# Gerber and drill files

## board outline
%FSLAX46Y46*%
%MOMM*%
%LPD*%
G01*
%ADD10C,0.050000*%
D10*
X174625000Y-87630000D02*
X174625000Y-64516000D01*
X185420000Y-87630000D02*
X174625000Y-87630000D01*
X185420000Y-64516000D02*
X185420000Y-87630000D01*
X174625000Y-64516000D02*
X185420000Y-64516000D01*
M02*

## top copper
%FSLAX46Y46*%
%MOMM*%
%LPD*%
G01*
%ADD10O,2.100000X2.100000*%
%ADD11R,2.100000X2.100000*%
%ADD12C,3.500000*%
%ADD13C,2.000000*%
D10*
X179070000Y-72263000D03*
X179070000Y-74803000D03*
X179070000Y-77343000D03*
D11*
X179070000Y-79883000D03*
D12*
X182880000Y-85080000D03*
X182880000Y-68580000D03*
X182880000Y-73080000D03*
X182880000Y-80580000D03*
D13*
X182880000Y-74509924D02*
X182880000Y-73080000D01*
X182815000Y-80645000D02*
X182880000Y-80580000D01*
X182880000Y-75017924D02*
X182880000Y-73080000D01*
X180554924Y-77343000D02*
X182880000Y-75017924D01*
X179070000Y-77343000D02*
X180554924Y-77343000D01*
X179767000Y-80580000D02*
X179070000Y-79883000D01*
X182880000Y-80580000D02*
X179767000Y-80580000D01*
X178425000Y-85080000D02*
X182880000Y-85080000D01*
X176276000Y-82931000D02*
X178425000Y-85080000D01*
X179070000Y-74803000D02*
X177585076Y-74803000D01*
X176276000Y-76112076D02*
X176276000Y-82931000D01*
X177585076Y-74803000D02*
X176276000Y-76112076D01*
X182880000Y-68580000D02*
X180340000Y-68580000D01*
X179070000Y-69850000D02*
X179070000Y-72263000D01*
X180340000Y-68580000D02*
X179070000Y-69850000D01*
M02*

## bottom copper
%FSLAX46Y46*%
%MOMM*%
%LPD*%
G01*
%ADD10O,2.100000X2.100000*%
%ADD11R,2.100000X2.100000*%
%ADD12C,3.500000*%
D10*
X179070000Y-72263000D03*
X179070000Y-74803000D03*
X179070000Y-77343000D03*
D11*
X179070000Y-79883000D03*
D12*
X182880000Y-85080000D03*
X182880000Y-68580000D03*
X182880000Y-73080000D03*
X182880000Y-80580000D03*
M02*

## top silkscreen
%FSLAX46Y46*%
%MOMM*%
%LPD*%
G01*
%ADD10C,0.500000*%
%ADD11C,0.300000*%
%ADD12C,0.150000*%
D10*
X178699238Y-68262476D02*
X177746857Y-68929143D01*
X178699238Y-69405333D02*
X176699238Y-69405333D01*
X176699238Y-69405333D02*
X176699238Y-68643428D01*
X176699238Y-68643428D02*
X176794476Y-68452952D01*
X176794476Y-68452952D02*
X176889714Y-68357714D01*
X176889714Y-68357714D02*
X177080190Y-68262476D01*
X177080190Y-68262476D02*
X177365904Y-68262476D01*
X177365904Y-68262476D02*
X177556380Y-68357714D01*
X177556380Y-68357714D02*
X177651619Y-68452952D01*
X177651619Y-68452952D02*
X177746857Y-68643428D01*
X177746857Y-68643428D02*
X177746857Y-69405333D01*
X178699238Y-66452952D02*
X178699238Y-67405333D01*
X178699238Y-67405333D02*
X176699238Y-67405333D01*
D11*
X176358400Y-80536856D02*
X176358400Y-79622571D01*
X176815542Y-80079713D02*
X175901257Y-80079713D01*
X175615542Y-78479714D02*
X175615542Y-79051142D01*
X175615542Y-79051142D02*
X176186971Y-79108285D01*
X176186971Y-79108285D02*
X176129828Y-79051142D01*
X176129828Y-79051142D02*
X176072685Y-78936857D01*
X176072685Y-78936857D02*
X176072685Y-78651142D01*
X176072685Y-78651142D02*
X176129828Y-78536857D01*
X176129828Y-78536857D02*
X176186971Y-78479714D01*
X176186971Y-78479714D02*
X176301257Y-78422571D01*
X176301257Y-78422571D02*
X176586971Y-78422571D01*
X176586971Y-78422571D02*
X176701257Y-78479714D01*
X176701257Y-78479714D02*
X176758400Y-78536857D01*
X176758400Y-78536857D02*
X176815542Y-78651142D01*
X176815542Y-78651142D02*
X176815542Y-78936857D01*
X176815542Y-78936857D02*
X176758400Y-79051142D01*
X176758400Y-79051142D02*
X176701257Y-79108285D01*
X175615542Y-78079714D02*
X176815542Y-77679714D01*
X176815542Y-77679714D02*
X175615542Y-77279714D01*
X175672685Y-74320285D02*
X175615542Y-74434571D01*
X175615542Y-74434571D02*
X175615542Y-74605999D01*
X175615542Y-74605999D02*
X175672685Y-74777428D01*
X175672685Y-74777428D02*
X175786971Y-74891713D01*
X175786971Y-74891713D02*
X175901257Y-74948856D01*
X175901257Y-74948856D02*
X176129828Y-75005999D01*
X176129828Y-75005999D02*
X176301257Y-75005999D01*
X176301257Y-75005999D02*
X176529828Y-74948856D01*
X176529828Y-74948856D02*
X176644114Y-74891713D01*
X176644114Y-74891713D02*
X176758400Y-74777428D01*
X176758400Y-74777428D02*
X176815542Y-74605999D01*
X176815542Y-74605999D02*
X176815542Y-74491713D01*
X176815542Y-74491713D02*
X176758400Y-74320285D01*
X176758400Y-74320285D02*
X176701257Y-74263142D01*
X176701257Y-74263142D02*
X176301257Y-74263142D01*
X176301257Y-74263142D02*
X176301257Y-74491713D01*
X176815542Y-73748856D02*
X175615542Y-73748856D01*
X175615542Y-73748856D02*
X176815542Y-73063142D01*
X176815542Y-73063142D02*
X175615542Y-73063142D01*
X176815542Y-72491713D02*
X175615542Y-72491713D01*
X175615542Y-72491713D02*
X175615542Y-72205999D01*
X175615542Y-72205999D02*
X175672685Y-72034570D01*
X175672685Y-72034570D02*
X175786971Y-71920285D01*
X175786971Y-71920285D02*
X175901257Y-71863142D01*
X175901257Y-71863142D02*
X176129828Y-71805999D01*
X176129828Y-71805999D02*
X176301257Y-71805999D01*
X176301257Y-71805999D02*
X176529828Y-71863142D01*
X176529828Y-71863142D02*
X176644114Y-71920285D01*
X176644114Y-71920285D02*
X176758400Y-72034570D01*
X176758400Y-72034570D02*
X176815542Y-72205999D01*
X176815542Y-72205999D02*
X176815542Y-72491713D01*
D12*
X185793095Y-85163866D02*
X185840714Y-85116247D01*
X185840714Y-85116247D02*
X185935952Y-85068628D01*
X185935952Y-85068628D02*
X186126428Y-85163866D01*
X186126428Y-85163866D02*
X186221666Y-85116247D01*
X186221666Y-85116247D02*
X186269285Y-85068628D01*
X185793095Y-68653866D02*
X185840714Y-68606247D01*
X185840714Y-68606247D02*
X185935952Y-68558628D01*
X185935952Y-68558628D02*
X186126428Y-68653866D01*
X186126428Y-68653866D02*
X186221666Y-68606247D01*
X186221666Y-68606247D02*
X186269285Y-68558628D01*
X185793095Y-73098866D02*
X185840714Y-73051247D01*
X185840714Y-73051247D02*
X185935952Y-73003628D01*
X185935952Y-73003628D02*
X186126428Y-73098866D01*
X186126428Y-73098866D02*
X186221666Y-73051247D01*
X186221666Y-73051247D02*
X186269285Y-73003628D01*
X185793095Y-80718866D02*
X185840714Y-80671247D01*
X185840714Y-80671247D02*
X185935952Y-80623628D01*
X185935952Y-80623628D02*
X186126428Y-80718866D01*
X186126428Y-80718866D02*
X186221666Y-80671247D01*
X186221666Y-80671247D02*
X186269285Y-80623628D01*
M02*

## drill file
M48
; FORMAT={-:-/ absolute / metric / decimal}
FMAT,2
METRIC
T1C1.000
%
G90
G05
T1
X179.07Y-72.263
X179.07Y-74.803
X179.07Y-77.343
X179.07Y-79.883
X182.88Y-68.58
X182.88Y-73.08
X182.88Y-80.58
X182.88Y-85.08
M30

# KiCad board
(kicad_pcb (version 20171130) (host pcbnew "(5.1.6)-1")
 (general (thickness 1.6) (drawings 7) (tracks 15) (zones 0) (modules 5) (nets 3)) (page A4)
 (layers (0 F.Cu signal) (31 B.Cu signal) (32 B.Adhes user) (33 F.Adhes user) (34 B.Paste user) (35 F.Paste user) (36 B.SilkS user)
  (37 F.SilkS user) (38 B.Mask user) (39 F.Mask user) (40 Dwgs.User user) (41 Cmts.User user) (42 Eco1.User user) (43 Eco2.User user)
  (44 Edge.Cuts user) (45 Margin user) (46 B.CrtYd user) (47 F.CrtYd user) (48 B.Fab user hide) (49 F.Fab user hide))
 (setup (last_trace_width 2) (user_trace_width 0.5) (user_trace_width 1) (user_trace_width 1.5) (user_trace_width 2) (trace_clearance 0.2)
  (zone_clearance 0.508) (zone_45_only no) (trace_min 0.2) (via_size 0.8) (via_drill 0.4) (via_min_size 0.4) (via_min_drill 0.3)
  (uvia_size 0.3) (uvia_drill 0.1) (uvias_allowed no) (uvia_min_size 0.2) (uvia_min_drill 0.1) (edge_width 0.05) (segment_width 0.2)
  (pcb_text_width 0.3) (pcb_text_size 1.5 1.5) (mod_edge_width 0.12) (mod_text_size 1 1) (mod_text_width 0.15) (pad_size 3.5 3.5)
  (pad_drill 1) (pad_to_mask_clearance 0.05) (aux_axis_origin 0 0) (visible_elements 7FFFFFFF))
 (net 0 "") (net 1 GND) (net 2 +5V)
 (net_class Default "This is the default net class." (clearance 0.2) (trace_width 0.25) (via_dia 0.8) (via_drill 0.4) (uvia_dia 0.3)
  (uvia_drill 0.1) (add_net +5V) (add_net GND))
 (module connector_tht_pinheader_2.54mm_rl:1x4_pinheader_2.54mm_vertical (layer B.Cu) (at 179.07 79.883)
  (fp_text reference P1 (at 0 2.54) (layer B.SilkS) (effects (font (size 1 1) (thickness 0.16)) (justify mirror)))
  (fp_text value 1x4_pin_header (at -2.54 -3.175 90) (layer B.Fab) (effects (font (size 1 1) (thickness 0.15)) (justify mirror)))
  (pad 4 thru_hole oval (at 0 -7.62) (size 2.1 2.1) (drill 1) (layers *.Cu *.Mask) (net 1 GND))
  (pad 3 thru_hole oval (at 0 -5.08) (size 2.1 2.1) (drill 1) (layers *.Cu *.Mask) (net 1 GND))
  (pad 2 thru_hole oval (at 0 -2.54) (size 2.1 2.1) (drill 1) (layers *.Cu *.Mask) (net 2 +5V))
  (pad 1 thru_hole rect (at 0 0) (size 2.1 2.1) (drill 1) (layers *.Cu *.Mask) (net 2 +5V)))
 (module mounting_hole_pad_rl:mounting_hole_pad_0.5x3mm (layer F.Cu) (at 182.88 85.08)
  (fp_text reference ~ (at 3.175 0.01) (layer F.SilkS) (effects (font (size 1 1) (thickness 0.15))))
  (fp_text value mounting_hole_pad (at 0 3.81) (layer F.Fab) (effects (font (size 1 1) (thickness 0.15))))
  (pad 1 thru_hole circle (at 0 0) (size 3.5 3.5) (drill 1) (layers *.Cu *.Mask) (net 1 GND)))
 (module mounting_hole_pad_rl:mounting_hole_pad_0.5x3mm (layer F.Cu) (at 182.88 68.58)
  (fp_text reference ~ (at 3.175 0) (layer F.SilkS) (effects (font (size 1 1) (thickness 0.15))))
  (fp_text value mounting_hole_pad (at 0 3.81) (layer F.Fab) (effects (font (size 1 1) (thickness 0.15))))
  (pad 1 thru_hole circle (at 0 0) (size 3.5 3.5) (drill 1) (layers *.Cu *.Mask) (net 1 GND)))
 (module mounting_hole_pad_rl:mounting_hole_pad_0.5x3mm (layer F.Cu) (at 182.88 73.08)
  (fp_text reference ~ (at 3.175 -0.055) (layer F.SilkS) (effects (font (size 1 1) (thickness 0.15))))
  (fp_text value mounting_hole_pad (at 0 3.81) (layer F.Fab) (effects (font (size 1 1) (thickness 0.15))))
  (pad 1 thru_hole circle (at 0 0) (size 3.5 3.5) (drill 1) (layers *.Cu *.Mask) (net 2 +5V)))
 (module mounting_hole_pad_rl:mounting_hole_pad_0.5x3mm (layer F.Cu) (at 182.88 80.58)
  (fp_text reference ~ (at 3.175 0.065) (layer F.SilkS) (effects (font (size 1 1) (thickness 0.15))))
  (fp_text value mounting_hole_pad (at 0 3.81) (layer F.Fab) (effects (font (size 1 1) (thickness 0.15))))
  (pad 1 thru_hole circle (at 0 0) (size 3.5 3.5) (drill 1) (layers *.Cu *.Mask) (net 2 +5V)))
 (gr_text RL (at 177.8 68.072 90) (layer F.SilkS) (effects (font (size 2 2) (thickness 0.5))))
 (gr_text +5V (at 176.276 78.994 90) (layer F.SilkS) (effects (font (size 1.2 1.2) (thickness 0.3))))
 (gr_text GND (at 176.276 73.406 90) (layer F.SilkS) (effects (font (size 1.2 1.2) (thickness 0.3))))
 (gr_line (start 174.625 87.63) (end 174.625 64.516) (layer Edge.Cuts) (width 0.05))
 (gr_line (start 185.42 87.63) (end 174.625 87.63) (layer Edge.Cuts) (width 0.05))
 (gr_line (start 185.42 64.516) (end 185.42 87.63) (layer Edge.Cuts) (width 0.05))
 (gr_line (start 174.625 64.516) (end 185.42 64.516) (layer Edge.Cuts) (width 0.05))
 (segment (start 182.88 74.509924) (end 182.88 73.08) (width 2) (layer F.Cu) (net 2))
 (segment (start 182.815 80.645) (end 182.88 80.58) (width 2) (layer F.Cu) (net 2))
 (segment (start 182.88 75.017924) (end 182.88 73.08) (width 2) (layer F.Cu) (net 2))
 (segment (start 180.554924 77.343) (end 182.88 75.017924) (width 2) (layer F.Cu) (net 2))
 (segment (start 179.07 77.343) (end 180.554924 77.343) (width 2) (layer F.Cu) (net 2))
 (segment (start 179.767 80.58) (end 179.07 79.883) (width 2) (layer F.Cu) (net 2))
 (segment (start 182.88 80.58) (end 179.767 80.58) (width 2) (layer F.Cu) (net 2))
 (segment (start 178.425 85.08) (end 182.88 85.08) (width 2) (layer F.Cu) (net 1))
 (segment (start 176.276 82.931) (end 178.425 85.08) (width 2) (layer F.Cu) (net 1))
 (segment (start 179.07 74.803) (end 177.585076 74.803) (width 2) (layer F.Cu) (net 1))
 (segment (start 176.276 76.112076) (end 176.276 82.931) (width 2) (layer F.Cu) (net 1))
 (segment (start 177.585076 74.803) (end 176.276 76.112076) (width 2) (layer F.Cu) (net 1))
 (segment (start 182.88 68.58) (end 180.34 68.58) (width 2) (layer F.Cu) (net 1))
 (segment (start 179.07 69.85) (end 179.07 72.263) (width 2) (layer F.Cu) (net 1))
 (segment (start 180.34 68.58) (end 179.07 69.85) (width 2) (layer F.Cu) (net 1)))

